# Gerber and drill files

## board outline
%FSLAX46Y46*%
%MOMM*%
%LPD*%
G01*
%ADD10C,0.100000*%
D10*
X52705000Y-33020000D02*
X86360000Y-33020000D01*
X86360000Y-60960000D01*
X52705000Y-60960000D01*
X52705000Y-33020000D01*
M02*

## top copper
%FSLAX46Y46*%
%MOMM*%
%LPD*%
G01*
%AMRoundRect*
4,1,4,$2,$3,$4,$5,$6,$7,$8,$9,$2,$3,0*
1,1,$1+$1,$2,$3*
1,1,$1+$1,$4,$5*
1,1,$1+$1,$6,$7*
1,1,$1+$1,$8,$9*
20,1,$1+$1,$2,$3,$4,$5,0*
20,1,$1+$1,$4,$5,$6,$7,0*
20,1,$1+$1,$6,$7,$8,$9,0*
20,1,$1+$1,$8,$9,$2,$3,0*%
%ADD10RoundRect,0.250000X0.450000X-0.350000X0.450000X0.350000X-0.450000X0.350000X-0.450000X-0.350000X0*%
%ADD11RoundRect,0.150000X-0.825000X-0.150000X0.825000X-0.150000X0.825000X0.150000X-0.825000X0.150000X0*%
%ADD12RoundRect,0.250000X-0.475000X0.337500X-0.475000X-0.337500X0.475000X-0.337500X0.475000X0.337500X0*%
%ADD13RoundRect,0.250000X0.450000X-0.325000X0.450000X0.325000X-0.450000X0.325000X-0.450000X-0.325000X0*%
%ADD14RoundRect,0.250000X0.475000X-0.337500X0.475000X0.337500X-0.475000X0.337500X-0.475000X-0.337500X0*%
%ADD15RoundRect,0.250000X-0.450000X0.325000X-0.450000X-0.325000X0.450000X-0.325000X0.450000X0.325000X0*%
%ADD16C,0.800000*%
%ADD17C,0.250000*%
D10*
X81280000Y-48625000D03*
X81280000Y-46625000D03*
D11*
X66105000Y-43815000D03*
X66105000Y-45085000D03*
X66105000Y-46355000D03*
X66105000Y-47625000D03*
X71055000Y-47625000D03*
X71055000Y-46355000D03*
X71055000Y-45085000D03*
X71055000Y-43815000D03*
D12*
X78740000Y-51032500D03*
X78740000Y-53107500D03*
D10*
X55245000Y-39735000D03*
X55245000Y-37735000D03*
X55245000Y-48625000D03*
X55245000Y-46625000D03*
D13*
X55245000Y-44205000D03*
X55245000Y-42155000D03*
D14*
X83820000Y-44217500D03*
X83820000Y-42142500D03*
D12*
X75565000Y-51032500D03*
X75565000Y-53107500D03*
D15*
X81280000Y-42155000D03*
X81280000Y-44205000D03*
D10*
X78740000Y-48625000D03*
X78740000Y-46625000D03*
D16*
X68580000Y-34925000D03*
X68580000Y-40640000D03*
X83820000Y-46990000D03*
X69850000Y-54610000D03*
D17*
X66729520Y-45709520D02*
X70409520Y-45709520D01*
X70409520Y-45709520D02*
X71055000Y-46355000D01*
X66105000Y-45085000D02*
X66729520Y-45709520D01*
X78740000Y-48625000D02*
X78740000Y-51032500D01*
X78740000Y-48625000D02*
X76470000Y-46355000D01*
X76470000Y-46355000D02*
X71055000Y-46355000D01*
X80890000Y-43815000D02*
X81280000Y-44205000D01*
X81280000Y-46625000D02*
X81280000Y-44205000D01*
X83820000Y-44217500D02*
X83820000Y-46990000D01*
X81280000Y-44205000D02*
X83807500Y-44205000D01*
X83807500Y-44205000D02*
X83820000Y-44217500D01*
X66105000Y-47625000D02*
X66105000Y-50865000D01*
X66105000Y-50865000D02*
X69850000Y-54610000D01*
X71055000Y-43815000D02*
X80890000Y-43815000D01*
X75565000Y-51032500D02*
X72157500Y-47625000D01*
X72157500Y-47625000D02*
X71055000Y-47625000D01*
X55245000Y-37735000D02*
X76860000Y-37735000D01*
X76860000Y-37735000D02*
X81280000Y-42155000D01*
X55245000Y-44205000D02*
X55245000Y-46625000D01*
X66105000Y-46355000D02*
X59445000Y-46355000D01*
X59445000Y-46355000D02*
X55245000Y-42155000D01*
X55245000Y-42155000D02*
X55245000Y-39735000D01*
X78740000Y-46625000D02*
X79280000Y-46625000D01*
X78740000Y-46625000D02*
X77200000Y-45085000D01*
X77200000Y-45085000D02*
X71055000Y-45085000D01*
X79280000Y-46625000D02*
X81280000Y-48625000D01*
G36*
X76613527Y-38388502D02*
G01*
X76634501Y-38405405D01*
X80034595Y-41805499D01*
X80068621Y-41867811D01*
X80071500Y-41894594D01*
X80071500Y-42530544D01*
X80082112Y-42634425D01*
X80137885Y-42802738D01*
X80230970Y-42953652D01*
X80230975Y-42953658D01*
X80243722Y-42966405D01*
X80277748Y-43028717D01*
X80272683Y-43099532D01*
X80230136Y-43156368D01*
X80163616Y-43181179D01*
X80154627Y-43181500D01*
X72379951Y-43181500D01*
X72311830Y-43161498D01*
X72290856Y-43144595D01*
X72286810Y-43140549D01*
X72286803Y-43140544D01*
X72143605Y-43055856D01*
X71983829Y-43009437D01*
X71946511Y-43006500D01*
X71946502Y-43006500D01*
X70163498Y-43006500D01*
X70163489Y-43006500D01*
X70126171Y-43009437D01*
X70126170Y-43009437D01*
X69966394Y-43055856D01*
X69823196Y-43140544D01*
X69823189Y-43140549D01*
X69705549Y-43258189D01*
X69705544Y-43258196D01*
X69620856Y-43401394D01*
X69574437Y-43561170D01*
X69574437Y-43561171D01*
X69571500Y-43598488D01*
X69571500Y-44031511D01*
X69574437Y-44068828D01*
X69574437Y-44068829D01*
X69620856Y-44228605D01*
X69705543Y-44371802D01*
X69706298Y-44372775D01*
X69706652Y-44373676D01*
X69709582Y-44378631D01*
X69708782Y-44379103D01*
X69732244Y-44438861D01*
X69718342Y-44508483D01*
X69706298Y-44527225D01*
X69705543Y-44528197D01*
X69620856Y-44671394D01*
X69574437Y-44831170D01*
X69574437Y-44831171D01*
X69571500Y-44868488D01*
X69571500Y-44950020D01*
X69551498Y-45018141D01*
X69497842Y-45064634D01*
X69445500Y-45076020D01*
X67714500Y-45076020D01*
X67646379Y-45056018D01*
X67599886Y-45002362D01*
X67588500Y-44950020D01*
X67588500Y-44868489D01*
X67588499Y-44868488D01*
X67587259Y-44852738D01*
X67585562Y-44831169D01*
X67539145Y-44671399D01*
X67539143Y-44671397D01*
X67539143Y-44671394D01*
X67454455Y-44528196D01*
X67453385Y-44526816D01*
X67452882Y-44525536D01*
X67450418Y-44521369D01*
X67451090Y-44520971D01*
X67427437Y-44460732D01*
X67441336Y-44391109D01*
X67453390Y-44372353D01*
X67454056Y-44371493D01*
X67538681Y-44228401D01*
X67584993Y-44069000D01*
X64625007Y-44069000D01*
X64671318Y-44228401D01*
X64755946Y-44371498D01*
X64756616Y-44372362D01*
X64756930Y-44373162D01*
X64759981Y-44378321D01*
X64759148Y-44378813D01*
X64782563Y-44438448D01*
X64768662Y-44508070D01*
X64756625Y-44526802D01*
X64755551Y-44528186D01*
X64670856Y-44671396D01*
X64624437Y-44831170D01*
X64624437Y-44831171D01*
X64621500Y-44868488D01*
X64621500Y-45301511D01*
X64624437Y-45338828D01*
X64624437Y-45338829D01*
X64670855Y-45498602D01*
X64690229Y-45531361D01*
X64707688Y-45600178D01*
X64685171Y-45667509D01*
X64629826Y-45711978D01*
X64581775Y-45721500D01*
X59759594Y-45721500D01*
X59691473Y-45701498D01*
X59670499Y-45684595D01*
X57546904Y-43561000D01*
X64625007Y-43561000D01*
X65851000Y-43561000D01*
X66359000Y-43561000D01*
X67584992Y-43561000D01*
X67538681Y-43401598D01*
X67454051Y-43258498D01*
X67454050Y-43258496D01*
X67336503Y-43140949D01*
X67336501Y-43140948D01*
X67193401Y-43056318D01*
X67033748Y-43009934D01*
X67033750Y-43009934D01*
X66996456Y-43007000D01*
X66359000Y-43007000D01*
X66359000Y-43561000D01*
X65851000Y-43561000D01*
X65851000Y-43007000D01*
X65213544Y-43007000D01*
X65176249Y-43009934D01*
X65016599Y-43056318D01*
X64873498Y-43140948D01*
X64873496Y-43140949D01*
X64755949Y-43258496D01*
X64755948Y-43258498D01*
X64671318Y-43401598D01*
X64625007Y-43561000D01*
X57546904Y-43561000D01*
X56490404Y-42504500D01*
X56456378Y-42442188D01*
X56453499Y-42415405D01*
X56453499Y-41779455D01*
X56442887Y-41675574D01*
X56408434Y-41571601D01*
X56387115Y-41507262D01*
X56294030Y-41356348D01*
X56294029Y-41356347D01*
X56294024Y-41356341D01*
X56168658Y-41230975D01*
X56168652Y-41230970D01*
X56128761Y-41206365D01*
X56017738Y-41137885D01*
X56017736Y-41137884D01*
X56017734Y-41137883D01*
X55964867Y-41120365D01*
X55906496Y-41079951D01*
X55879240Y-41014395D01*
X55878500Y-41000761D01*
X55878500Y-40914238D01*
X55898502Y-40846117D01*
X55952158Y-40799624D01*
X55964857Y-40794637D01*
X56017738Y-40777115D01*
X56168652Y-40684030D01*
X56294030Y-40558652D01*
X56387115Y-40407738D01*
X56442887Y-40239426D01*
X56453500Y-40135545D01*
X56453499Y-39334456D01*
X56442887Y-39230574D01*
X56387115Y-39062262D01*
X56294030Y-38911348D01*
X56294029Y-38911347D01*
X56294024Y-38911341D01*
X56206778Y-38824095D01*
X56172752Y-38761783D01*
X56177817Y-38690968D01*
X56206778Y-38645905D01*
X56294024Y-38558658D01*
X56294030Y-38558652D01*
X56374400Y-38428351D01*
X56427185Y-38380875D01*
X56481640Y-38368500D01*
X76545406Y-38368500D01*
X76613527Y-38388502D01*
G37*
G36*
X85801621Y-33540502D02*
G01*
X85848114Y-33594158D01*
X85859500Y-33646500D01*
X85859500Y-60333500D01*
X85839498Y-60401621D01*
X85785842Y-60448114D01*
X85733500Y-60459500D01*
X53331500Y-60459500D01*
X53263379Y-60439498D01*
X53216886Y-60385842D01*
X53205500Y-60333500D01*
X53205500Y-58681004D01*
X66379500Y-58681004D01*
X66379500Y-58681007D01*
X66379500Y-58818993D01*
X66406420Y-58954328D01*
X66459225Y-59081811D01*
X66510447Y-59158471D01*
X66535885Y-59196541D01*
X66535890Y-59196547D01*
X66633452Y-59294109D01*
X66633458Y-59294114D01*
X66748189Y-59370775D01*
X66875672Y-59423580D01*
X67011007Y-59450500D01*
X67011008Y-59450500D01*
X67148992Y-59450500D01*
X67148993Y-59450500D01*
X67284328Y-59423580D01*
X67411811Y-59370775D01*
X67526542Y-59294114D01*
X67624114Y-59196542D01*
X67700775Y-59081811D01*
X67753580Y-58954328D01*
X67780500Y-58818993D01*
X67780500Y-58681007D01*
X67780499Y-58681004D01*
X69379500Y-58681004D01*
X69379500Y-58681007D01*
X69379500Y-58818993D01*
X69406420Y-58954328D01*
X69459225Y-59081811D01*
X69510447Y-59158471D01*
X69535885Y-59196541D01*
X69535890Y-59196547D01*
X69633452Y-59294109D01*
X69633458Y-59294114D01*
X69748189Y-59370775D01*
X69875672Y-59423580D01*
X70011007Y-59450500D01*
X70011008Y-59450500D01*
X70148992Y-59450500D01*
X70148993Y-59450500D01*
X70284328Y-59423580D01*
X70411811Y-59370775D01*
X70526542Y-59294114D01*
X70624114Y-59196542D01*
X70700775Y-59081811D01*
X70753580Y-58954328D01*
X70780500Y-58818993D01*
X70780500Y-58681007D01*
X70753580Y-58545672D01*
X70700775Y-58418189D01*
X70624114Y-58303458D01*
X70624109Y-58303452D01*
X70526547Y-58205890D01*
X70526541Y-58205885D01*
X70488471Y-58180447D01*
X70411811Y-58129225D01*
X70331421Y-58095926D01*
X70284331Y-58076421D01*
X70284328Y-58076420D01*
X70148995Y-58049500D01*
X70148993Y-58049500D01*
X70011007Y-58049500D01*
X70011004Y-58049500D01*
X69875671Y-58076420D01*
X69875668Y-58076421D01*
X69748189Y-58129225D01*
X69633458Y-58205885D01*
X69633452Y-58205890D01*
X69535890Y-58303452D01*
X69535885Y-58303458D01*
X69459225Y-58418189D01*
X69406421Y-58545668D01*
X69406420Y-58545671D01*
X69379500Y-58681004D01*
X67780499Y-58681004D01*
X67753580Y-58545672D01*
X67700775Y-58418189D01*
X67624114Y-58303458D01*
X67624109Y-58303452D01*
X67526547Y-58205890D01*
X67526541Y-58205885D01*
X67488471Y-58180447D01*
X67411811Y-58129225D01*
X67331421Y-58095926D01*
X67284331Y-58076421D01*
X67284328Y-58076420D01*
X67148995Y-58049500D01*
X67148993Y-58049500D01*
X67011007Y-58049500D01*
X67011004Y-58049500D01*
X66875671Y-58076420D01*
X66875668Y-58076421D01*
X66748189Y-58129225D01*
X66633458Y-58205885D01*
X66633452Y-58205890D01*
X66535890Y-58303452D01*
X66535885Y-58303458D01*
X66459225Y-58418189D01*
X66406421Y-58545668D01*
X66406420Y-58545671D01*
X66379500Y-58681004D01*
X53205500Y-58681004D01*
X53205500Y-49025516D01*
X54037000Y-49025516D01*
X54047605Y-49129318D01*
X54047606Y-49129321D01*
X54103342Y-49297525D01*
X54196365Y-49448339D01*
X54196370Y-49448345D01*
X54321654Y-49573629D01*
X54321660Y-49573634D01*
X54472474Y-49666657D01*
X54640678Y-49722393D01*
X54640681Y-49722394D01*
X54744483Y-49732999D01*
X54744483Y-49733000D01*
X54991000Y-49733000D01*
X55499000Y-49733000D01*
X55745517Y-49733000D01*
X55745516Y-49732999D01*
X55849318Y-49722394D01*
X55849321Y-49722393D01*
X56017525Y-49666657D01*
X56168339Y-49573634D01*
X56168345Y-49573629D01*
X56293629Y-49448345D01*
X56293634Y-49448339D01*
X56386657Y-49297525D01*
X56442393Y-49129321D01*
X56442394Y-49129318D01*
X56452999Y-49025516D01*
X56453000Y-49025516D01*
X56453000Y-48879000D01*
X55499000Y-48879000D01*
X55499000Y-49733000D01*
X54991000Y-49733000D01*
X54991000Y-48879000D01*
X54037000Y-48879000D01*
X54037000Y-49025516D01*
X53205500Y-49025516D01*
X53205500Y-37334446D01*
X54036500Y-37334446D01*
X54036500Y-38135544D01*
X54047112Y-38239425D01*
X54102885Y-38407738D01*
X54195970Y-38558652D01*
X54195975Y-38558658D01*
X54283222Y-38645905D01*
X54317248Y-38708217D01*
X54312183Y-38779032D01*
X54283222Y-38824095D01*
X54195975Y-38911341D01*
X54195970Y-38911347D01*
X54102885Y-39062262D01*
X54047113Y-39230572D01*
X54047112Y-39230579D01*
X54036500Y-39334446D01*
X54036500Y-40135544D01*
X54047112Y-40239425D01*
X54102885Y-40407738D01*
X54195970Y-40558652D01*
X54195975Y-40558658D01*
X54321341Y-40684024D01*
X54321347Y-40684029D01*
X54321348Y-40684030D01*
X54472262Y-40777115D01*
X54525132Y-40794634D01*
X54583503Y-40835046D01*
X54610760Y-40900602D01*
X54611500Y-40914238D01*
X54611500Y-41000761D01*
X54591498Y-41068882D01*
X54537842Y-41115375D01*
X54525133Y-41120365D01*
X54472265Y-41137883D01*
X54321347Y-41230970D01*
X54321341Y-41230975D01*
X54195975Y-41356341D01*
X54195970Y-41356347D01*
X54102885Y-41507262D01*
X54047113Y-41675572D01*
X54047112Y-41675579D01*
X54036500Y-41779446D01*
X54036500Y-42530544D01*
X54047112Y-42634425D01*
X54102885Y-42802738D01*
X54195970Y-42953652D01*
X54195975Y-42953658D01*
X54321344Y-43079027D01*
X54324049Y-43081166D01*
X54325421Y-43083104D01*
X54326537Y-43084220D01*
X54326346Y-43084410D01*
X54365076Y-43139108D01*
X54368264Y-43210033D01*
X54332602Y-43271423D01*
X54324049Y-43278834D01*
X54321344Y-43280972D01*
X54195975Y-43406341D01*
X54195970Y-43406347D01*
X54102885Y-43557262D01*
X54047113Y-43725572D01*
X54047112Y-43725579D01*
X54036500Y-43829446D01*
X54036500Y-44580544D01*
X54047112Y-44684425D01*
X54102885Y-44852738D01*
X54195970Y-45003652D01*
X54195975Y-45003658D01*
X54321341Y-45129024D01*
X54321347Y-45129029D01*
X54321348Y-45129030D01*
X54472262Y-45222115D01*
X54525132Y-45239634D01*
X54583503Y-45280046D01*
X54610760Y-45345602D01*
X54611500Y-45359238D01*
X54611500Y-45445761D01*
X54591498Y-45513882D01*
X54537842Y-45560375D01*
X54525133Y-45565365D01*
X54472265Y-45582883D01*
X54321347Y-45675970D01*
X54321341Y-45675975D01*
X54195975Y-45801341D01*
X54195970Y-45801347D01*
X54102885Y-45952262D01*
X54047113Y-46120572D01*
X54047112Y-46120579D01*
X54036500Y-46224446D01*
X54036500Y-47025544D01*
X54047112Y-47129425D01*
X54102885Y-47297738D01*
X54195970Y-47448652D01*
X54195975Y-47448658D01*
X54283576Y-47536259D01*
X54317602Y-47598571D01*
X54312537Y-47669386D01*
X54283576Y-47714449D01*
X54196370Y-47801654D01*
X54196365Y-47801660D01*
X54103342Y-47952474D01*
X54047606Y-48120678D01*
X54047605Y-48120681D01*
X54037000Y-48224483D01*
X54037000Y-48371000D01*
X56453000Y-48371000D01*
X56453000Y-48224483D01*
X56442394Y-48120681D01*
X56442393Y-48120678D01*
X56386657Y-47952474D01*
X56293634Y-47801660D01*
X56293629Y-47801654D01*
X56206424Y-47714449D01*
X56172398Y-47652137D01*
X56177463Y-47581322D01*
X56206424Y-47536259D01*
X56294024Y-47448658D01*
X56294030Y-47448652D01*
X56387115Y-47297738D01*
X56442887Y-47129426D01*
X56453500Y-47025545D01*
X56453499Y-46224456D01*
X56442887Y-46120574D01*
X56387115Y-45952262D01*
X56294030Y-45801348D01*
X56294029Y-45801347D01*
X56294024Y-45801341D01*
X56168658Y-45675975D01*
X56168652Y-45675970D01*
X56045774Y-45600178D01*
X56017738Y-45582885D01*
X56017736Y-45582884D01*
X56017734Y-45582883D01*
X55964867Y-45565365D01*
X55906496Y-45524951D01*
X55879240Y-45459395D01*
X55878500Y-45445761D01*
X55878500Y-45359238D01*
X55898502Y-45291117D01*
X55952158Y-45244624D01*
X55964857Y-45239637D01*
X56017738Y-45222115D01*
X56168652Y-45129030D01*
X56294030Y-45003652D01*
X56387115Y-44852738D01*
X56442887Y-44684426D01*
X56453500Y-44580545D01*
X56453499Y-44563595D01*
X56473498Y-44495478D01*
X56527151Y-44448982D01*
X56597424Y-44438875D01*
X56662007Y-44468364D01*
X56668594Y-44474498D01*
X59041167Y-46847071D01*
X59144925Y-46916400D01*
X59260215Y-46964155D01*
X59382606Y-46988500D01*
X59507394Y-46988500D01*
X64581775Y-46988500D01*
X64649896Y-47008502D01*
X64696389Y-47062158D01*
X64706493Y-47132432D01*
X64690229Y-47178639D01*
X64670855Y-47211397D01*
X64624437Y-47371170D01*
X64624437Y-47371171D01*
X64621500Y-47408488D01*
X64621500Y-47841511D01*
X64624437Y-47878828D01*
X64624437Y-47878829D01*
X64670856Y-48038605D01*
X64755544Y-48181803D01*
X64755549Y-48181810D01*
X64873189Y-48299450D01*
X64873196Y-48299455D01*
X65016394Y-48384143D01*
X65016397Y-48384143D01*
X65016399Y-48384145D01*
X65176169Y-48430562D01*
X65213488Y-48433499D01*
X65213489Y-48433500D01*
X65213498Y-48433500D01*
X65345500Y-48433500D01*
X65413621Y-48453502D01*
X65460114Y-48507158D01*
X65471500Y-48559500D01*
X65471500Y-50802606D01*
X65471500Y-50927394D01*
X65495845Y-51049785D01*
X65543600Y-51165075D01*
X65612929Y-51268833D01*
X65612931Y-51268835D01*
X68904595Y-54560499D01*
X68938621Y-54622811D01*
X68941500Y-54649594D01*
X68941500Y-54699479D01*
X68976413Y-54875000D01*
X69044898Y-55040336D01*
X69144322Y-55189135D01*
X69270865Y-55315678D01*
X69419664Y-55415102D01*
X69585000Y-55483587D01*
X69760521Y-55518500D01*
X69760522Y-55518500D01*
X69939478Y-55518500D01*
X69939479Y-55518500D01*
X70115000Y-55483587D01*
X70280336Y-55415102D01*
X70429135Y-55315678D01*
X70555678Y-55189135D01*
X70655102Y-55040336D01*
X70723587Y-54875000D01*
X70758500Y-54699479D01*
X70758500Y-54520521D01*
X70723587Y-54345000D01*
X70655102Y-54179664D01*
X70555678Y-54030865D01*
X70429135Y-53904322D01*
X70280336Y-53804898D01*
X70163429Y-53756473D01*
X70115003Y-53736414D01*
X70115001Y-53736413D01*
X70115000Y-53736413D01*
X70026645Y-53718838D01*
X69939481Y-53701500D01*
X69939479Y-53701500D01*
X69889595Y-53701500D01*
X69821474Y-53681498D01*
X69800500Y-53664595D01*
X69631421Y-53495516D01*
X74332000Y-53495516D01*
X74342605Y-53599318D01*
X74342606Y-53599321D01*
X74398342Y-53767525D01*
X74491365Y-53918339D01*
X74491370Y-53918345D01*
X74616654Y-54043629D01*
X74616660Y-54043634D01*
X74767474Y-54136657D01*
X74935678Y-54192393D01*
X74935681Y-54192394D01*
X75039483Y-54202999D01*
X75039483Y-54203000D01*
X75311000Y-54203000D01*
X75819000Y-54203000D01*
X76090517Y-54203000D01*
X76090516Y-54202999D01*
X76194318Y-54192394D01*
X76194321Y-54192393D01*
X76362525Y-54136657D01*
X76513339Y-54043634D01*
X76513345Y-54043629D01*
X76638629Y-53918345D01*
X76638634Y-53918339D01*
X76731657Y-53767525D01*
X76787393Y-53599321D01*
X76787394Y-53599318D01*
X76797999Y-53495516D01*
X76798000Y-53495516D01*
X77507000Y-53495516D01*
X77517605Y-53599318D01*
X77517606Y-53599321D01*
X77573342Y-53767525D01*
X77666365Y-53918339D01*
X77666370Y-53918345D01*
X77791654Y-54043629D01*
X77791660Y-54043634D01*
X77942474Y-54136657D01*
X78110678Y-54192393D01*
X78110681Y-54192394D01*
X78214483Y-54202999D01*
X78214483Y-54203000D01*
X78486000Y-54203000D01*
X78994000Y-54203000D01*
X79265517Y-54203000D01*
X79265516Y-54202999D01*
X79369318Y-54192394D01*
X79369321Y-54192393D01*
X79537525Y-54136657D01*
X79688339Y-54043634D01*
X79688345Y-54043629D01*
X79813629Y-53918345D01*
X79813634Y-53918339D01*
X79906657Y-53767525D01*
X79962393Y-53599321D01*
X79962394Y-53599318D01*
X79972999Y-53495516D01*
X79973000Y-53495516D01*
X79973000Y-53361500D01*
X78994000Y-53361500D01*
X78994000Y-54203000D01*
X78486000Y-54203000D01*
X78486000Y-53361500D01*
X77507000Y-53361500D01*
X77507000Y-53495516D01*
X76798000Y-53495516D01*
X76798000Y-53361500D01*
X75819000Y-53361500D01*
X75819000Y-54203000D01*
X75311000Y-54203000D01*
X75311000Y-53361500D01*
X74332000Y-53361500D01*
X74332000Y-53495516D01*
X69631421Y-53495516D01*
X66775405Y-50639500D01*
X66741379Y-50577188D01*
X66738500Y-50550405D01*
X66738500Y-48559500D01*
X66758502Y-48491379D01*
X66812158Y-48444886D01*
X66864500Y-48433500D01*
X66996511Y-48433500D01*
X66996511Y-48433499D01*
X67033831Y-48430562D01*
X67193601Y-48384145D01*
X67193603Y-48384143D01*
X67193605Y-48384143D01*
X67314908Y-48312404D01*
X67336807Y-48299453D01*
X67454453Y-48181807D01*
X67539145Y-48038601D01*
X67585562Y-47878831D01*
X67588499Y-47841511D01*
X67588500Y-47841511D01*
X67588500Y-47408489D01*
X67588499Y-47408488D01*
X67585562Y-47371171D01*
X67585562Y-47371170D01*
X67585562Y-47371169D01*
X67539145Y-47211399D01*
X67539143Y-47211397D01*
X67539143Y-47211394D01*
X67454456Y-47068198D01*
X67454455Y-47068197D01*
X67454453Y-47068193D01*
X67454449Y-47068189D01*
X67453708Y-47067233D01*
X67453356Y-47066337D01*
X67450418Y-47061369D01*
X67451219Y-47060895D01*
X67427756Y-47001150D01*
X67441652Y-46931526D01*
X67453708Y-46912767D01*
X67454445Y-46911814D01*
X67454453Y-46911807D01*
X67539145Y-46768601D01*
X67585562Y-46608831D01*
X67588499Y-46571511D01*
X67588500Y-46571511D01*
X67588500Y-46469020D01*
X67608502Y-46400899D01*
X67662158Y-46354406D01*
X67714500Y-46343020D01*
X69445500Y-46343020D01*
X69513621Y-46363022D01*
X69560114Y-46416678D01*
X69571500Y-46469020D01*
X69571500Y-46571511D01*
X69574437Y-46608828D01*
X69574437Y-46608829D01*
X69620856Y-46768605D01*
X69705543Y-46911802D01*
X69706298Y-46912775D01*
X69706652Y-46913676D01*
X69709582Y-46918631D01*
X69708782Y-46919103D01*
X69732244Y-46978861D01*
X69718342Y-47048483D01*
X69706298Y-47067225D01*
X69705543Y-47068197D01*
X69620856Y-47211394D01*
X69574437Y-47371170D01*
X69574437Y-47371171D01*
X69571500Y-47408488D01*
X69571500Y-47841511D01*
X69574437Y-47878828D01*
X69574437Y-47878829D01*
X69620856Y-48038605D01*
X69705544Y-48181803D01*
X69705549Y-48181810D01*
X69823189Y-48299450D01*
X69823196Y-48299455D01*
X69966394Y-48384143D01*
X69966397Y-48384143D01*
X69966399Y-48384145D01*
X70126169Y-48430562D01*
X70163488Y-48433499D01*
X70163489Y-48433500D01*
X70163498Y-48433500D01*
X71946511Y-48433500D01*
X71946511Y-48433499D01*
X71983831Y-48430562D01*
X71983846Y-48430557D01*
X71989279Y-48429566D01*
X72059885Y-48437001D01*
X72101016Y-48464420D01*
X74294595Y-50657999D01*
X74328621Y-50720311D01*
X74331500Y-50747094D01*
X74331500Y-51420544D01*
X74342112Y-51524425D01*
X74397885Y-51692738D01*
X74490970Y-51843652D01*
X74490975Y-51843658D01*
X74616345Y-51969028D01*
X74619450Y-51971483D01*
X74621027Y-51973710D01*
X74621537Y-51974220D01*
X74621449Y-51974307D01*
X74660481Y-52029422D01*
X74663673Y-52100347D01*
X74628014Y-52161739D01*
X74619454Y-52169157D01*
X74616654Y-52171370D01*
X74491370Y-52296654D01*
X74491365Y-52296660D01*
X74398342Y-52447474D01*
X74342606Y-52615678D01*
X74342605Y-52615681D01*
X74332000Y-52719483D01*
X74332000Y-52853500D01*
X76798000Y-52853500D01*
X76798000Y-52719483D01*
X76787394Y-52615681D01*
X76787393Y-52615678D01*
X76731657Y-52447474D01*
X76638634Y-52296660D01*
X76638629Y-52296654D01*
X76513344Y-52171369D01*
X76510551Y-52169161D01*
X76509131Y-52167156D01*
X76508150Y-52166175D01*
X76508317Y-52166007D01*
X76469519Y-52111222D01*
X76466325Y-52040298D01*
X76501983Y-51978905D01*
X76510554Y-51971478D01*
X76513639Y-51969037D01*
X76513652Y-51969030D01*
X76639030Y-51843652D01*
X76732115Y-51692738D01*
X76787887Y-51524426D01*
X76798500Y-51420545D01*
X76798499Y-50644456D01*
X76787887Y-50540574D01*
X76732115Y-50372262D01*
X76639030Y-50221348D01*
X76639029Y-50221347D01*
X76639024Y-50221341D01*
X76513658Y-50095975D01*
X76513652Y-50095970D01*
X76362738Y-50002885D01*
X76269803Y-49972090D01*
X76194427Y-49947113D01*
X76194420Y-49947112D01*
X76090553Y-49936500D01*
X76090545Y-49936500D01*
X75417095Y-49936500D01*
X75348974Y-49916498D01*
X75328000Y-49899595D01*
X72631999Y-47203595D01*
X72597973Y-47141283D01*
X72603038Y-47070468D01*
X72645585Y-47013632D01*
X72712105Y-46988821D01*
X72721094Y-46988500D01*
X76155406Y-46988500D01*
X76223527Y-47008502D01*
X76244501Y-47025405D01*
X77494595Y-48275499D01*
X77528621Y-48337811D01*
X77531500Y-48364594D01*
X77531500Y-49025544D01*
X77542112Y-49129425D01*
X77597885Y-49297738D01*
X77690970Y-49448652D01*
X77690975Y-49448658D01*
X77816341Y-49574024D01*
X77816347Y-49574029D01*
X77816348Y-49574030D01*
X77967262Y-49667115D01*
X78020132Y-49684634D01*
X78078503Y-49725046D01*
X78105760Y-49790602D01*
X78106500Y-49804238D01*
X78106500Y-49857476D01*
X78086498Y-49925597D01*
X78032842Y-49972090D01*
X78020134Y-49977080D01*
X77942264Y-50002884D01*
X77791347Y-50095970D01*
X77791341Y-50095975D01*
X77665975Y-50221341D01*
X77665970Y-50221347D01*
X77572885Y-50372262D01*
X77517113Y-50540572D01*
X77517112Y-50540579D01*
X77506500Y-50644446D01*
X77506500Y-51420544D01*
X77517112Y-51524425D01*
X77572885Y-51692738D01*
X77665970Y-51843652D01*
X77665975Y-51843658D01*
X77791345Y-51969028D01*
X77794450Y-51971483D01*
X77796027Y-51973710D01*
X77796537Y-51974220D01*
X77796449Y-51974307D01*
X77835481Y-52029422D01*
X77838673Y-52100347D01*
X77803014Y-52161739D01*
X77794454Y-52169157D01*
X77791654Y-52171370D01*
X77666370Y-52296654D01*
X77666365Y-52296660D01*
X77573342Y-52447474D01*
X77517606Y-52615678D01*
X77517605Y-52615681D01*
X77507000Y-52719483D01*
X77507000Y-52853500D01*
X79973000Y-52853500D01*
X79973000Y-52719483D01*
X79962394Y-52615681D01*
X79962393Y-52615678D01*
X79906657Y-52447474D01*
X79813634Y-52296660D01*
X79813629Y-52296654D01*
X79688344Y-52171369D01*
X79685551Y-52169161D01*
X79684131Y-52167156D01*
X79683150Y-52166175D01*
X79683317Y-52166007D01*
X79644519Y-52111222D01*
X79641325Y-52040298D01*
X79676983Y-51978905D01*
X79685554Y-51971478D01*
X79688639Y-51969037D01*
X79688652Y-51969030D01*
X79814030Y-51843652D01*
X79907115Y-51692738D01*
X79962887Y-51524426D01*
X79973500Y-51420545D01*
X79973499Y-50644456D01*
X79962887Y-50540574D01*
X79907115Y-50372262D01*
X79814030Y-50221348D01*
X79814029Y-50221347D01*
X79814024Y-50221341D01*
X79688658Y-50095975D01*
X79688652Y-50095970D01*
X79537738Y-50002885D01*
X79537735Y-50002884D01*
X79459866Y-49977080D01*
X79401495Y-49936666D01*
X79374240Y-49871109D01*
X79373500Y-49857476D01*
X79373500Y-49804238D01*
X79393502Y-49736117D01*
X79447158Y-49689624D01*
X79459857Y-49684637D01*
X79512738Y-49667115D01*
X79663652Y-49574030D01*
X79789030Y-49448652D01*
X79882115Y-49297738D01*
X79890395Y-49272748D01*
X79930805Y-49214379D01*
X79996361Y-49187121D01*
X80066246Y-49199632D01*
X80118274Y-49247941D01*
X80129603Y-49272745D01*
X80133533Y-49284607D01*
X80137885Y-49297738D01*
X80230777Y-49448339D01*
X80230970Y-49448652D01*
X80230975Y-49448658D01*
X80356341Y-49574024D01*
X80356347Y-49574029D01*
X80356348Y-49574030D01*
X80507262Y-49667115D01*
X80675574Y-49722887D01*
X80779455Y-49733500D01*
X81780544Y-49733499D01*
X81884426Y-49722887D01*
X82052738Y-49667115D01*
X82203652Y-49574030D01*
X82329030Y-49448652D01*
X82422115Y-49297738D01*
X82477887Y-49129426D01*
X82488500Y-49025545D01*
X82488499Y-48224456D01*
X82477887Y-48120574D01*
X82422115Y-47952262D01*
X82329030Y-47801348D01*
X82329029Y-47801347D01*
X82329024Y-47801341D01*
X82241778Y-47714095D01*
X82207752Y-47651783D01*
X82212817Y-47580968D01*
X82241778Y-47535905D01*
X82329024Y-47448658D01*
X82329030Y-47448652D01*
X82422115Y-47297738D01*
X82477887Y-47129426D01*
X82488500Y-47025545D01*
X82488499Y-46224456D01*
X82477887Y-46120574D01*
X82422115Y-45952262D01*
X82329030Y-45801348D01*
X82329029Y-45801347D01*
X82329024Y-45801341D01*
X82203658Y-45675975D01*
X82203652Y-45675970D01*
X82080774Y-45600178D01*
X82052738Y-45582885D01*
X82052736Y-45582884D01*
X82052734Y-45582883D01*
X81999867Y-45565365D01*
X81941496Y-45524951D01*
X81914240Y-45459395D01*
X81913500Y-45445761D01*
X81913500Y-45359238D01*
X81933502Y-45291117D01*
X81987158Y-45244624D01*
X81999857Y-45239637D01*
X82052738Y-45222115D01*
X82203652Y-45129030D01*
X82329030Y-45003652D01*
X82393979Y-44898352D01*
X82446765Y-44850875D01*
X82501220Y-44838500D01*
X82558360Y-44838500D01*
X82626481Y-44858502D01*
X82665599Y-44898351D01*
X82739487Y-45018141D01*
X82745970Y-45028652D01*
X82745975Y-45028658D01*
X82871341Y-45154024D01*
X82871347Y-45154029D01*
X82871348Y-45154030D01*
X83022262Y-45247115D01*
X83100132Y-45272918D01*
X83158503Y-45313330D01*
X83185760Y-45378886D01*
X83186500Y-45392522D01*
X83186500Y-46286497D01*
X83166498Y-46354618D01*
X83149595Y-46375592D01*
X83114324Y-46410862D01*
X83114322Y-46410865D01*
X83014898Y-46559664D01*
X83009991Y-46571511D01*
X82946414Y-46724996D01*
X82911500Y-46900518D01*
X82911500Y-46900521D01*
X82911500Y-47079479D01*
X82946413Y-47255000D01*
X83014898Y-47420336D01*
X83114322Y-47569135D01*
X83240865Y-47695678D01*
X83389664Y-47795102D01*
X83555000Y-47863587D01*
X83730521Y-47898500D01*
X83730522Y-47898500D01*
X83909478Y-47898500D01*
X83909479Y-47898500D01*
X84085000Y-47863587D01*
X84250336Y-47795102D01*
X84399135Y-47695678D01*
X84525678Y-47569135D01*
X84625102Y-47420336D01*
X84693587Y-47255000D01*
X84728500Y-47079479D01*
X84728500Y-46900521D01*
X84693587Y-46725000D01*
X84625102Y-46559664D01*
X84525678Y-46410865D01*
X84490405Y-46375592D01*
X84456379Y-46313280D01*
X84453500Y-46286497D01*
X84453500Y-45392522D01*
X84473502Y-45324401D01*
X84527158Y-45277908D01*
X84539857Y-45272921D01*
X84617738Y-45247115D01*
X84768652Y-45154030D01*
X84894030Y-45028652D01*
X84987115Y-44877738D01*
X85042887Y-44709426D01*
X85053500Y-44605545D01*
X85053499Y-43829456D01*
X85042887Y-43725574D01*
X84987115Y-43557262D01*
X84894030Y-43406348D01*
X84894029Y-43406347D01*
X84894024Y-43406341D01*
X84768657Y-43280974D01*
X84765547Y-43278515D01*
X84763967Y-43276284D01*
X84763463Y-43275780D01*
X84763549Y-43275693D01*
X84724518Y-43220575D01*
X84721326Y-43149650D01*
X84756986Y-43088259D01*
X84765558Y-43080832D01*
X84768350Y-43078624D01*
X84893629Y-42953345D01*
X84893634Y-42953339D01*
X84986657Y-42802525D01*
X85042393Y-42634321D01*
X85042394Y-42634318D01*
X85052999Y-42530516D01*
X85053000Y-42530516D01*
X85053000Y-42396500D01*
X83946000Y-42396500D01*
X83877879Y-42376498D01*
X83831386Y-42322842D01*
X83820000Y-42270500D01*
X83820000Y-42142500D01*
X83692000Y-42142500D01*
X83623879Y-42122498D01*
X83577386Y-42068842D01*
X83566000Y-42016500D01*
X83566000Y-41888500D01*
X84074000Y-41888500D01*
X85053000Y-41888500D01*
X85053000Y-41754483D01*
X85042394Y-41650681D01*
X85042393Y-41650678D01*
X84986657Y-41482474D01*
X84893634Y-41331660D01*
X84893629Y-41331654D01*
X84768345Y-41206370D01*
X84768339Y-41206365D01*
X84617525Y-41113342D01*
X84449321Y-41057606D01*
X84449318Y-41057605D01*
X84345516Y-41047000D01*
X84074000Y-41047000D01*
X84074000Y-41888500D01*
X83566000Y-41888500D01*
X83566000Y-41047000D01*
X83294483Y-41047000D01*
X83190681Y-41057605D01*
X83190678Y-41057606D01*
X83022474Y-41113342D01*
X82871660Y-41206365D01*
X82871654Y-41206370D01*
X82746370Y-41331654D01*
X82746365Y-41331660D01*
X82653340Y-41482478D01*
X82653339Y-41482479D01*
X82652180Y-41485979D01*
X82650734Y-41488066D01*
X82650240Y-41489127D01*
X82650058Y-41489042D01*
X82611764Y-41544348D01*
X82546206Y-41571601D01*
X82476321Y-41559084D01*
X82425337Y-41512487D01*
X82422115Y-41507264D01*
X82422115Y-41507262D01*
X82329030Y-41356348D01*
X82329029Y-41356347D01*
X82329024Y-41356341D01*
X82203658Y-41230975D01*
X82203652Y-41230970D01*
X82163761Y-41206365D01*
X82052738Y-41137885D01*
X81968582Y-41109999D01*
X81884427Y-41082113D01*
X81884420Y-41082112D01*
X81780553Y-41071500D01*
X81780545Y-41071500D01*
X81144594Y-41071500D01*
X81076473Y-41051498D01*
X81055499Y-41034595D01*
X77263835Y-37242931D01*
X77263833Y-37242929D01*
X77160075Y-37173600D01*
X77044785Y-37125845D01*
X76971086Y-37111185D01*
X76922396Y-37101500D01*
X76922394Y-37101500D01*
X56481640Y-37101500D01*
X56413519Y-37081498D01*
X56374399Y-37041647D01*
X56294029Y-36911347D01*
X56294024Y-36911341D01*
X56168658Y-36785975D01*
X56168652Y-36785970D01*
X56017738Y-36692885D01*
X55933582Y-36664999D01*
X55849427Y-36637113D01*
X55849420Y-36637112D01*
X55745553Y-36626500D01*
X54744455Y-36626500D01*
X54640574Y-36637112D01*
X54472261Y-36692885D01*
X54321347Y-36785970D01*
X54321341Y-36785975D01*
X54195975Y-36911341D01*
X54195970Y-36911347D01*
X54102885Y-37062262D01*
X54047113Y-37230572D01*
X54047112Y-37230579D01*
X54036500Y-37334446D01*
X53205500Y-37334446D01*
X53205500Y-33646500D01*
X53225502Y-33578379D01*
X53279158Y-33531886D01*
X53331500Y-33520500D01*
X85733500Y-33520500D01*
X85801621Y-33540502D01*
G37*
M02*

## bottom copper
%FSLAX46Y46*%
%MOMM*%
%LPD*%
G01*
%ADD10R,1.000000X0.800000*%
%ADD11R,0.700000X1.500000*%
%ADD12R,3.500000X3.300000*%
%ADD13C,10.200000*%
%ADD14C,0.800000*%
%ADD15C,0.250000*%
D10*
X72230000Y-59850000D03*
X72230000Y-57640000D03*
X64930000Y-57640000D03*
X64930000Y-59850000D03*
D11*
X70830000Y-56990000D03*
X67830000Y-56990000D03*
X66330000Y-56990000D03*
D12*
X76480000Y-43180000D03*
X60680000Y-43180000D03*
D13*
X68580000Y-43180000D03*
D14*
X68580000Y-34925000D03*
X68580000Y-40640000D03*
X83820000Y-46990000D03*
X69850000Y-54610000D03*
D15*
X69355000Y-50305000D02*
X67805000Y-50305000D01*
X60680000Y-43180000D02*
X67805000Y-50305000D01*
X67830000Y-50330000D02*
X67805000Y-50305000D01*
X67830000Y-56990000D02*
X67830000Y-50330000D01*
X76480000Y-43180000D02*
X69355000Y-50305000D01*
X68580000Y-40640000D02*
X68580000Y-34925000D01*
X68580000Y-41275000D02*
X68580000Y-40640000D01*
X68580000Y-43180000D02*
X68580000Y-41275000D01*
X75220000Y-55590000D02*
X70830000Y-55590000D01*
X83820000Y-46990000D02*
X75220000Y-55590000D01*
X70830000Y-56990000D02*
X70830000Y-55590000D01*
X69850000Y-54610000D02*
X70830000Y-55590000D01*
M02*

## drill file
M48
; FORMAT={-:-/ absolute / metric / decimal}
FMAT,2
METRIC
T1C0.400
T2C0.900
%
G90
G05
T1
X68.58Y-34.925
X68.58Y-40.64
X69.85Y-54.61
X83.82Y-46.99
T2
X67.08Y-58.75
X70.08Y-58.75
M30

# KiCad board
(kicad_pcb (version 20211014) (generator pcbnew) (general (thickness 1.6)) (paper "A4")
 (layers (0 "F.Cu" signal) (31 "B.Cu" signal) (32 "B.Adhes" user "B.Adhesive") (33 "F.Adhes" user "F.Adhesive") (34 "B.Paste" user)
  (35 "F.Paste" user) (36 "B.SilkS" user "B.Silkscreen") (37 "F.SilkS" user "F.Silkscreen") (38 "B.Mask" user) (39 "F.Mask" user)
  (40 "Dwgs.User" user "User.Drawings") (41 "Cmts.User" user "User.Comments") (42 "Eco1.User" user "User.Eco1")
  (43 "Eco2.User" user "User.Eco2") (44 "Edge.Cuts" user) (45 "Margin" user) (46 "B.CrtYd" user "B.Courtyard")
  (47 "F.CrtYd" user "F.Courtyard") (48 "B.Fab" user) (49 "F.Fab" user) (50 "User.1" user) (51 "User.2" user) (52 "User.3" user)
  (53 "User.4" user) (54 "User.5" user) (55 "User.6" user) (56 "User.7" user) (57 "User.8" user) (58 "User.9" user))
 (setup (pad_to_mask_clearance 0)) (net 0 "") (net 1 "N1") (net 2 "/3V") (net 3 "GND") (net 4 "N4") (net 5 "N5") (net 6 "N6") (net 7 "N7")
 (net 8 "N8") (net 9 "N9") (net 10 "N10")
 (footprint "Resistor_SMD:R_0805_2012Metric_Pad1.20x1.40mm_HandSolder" (layer "F.Cu") (at 81.28 47.625 90)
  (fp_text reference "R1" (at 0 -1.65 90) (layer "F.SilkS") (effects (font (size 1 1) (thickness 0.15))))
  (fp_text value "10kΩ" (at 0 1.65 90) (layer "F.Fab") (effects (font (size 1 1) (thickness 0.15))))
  (pad "1" smd roundrect (at -1 0 90) (size 1.2 1.4) (layers "F.Cu" "F.Paste" "F.Mask") (roundrect_rratio 0.208333) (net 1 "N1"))
  (pad "2" smd roundrect (at 1 0 90) (size 1.2 1.4) (layers "F.Cu" "F.Paste" "F.Mask") (roundrect_rratio 0.208333) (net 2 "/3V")))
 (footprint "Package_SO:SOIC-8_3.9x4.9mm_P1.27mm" (layer "F.Cu") (at 68.58 45.72)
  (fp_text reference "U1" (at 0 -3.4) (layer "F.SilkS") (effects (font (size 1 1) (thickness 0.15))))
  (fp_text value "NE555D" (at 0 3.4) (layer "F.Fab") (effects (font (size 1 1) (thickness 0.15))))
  (pad "1" smd roundrect (at -2.475 -1.905) (size 1.95 0.6) (layers "F.Cu" "F.Paste" "F.Mask") (roundrect_rratio 0.25) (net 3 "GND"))
  (pad "2" smd roundrect (at -2.475 -0.635) (size 1.95 0.6) (layers "F.Cu" "F.Paste" "F.Mask") (roundrect_rratio 0.25) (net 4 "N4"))
  (pad "3" smd roundrect (at -2.475 0.635) (size 1.95 0.6) (layers "F.Cu" "F.Paste" "F.Mask") (roundrect_rratio 0.25) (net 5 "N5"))
  (pad "4" smd roundrect (at -2.475 1.905) (size 1.95 0.6) (layers "F.Cu" "F.Paste" "F.Mask") (roundrect_rratio 0.25) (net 2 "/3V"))
  (pad "5" smd roundrect (at 2.475 1.905) (size 1.95 0.6) (layers "F.Cu" "F.Paste" "F.Mask") (roundrect_rratio 0.25) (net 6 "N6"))
  (pad "6" smd roundrect (at 2.475 0.635) (size 1.95 0.6) (layers "F.Cu" "F.Paste" "F.Mask") (roundrect_rratio 0.25) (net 4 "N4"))
  (pad "7" smd roundrect (at 2.475 -0.635) (size 1.95 0.6) (layers "F.Cu" "F.Paste" "F.Mask") (roundrect_rratio 0.25) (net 1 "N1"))
  (pad "8" smd roundrect (at 2.475 -1.905) (size 1.95 0.6) (layers "F.Cu" "F.Paste" "F.Mask") (roundrect_rratio 0.25) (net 2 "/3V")))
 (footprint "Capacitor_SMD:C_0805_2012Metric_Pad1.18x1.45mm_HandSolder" (layer "F.Cu") (at 78.74 52.07 -90)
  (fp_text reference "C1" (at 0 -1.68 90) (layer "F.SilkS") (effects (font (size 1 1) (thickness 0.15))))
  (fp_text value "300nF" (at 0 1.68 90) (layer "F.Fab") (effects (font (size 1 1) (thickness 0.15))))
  (pad "1" smd roundrect (at -1.0375 0 270) (size 1.175 1.45) (layers "F.Cu" "F.Paste" "F.Mask") (roundrect_rratio 0.212766) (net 4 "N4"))
  (pad "2" smd roundrect (at 1.0375 0 270) (size 1.175 1.45) (layers "F.Cu" "F.Paste" "F.Mask") (roundrect_rratio 0.212766) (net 3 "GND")))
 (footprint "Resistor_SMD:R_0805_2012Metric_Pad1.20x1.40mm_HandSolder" (layer "F.Cu") (at 55.245 38.735 90)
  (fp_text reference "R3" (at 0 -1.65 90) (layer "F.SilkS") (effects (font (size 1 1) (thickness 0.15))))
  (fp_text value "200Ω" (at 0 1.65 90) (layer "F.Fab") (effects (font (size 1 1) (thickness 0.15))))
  (pad "1" smd roundrect (at -1 0 90) (size 1.2 1.4) (layers "F.Cu" "F.Paste" "F.Mask") (roundrect_rratio 0.208333) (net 5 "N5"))
  (pad "2" smd roundrect (at 1 0 90) (size 1.2 1.4) (layers "F.Cu" "F.Paste" "F.Mask") (roundrect_rratio 0.208333) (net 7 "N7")))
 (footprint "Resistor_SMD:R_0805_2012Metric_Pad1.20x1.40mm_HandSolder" (layer "F.Cu") (at 55.245 47.625 90)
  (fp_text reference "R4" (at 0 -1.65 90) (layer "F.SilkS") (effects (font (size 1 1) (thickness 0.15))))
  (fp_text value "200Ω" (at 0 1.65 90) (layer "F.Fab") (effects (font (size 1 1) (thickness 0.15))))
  (pad "1" smd roundrect (at -1 0 90) (size 1.2 1.4) (layers "F.Cu" "F.Paste" "F.Mask") (roundrect_rratio 0.208333) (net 3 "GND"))
  (pad "2" smd roundrect (at 1 0 90) (size 1.2 1.4) (layers "F.Cu" "F.Paste" "F.Mask") (roundrect_rratio 0.208333) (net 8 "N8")))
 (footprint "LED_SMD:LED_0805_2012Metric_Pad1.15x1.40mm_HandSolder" (layer "F.Cu") (at 55.245 43.18 90)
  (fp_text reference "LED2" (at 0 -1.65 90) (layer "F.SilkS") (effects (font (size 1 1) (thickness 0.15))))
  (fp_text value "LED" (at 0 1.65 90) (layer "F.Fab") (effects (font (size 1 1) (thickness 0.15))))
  (pad "1" smd roundrect (at -1.025 0 90) (size 1.15 1.4) (layers "F.Cu" "F.Paste" "F.Mask") (roundrect_rratio 0.217391) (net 8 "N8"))
  (pad "2" smd roundrect (at 1.025 0 90) (size 1.15 1.4) (layers "F.Cu" "F.Paste" "F.Mask") (roundrect_rratio 0.217391) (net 5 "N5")))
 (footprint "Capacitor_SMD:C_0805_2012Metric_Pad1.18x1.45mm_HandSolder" (layer "F.Cu") (at 83.82 43.18 90)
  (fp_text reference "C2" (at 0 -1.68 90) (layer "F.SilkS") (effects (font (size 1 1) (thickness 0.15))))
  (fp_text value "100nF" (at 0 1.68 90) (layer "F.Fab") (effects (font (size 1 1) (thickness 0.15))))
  (pad "1" smd roundrect (at -1.0375 0 90) (size 1.175 1.45) (layers "F.Cu" "F.Paste" "F.Mask") (roundrect_rratio 0.212766) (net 2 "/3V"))
  (pad "2" smd roundrect (at 1.0375 0 90) (size 1.175 1.45) (layers "F.Cu" "F.Paste" "F.Mask") (roundrect_rratio 0.212766) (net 3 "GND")))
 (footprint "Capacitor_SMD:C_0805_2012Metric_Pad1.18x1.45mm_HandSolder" (layer "F.Cu") (at 75.565 52.07 -90)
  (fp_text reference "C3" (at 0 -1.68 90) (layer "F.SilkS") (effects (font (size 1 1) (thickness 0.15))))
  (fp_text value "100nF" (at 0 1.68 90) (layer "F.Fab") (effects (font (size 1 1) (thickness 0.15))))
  (pad "1" smd roundrect (at -1.0375 0 270) (size 1.175 1.45) (layers "F.Cu" "F.Paste" "F.Mask") (roundrect_rratio 0.212766) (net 6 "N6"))
  (pad "2" smd roundrect (at 1.0375 0 270) (size 1.175 1.45) (layers "F.Cu" "F.Paste" "F.Mask") (roundrect_rratio 0.212766) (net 3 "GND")))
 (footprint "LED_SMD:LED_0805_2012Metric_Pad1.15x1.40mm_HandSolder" (layer "F.Cu") (at 81.28 43.18 -90)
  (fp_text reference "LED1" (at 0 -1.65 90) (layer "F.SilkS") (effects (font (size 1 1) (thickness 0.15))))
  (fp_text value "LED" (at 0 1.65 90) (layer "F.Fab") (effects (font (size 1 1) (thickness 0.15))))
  (pad "1" smd roundrect (at -1.025 0 270) (size 1.15 1.4) (layers "F.Cu" "F.Paste" "F.Mask") (roundrect_rratio 0.217391) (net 7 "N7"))
  (pad "2" smd roundrect (at 1.025 0 270) (size 1.15 1.4) (layers "F.Cu" "F.Paste" "F.Mask") (roundrect_rratio 0.217391) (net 2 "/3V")))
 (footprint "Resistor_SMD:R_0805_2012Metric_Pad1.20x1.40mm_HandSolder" (layer "F.Cu") (at 78.74 47.625 90)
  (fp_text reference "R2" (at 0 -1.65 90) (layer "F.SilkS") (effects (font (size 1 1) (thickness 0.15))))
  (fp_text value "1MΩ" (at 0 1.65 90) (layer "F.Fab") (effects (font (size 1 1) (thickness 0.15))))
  (pad "1" smd roundrect (at -1 0 90) (size 1.2 1.4) (layers "F.Cu" "F.Paste" "F.Mask") (roundrect_rratio 0.208333) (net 4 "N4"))
  (pad "2" smd roundrect (at 1 0 90) (size 1.2 1.4) (layers "F.Cu" "F.Paste" "F.Mask") (roundrect_rratio 0.208333) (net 1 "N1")))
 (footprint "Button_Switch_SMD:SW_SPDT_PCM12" (layer "B.Cu") (at 68.58 58.42 180)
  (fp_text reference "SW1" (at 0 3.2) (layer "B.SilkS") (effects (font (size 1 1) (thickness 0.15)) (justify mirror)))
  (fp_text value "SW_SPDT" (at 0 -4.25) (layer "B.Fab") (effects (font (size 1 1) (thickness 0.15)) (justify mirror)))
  (pad "" smd rect (at -3.65 -1.43 180) (size 1 0.8) (layers "B.Cu" "B.Paste" "B.Mask"))
  (pad "" smd rect (at -3.65 0.78 180) (size 1 0.8) (layers "B.Cu" "B.Paste" "B.Mask"))
  (pad "" np_thru_hole circle (at -1.5 -0.33 180) (size 0.9 0.9) (drill 0.9) (layers *.Cu *.Mask))
  (pad "" smd rect (at 3.65 0.78 180) (size 1 0.8) (layers "B.Cu" "B.Paste" "B.Mask"))
  (pad "" smd rect (at 3.65 -1.43 180) (size 1 0.8) (layers "B.Cu" "B.Paste" "B.Mask"))
  (pad "" np_thru_hole circle (at 1.5 -0.33 180) (size 0.9 0.9) (drill 0.9) (layers *.Cu *.Mask))
  (pad "1" smd rect (at -2.25 1.43 180) (size 0.7 1.5) (layers "B.Cu" "B.Paste" "B.Mask") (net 2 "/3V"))
  (pad "2" smd rect (at 0.75 1.43 180) (size 0.7 1.5) (layers "B.Cu" "B.Paste" "B.Mask") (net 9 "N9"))
  (pad "3" smd rect (at 2.25 1.43 180) (size 0.7 1.5) (layers "B.Cu" "B.Paste" "B.Mask") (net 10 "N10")))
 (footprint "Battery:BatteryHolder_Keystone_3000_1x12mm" (layer "B.Cu") (at 68.58 43.18 180)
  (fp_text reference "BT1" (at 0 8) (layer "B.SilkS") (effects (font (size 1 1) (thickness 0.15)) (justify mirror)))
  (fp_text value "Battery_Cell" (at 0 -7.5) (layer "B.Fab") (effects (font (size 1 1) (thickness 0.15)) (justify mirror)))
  (pad "1" smd rect (at -7.9 0 180) (size 3.5 3.3) (layers "B.Cu" "B.Paste" "B.Mask") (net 9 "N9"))
  (pad "1" smd rect (at 7.9 0 180) (size 3.5 3.3) (layers "B.Cu" "B.Paste" "B.Mask") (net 9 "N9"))
  (pad "2" smd circle (at 0 0 180) (size 10.2 10.2) (layers "B.Cu" "B.Mask") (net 3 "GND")))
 (gr_rect (start 52.705 33.02) (end 86.36 60.96) (layer "Edge.Cuts") (width 0.1) (fill none))
 (segment (start 69.355 50.305) (end 67.805 50.305) (width 0.25) (layer "B.Cu") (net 9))
 (segment (start 60.68 43.18) (end 67.805 50.305) (width 0.25) (layer "B.Cu") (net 9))
 (segment (start 67.83 50.33) (end 67.805 50.305) (width 0.25) (layer "B.Cu") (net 9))
 (segment (start 67.83 56.99) (end 67.83 50.33) (width 0.25) (layer "B.Cu") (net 9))
 (segment (start 76.48 43.18) (end 69.355 50.305) (width 0.25) (layer "B.Cu") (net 9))
 (via (at 68.58 34.925) (size 0.8) (drill 0.4) (layers "F.Cu" "B.Cu") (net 3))
 (via (at 68.58 40.64) (size 0.8) (drill 0.4) (layers "F.Cu" "B.Cu") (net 3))
 (segment (start 68.58 40.64) (end 68.58 34.925) (width 0.25) (layer "B.Cu") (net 3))
 (segment (start 68.58 41.275) (end 68.58 40.64) (width 0.25) (layer "B.Cu") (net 3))
 (segment (start 68.58 43.18) (end 68.58 41.275) (width 0.25) (layer "B.Cu") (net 3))
 (segment (start 66.72952 45.70952) (end 70.40952 45.70952) (width 0.25) (layer "F.Cu") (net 4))
 (segment (start 70.40952 45.70952) (end 71.055 46.355) (width 0.25) (layer "F.Cu") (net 4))
 (segment (start 66.105 45.085) (end 66.72952 45.70952) (width 0.25) (layer "F.Cu") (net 4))
 (segment (start 78.74 48.625) (end 78.74 51.0325) (width 0.25) (layer "F.Cu") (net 4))
 (segment (start 78.74 48.625) (end 76.47 46.355) (width 0.25) (layer "F.Cu") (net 4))
 (segment (start 76.47 46.355) (end 71.055 46.355) (width 0.25) (layer "F.Cu") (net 4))
 (segment (start 80.89 43.815) (end 81.28 44.205) (width 0.25) (layer "F.Cu") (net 2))
 (segment (start 81.28 46.625) (end 81.28 44.205) (width 0.25) (layer "F.Cu") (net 2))
 (segment (start 83.82 44.2175) (end 83.82 46.99) (width 0.25) (layer "F.Cu") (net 2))
 (segment (start 81.28 44.205) (end 83.8075 44.205) (width 0.25) (layer "F.Cu") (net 2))
 (segment (start 83.8075 44.205) (end 83.82 44.2175) (width 0.25) (layer "F.Cu") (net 2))
 (segment (start 66.105 47.625) (end 66.105 50.865) (width 0.25) (layer "F.Cu") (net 2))
 (segment (start 66.105 50.865) (end 69.85 54.61) (width 0.25) (layer "F.Cu") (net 2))
 (segment (start 71.055 43.815) (end 80.89 43.815) (width 0.25) (layer "F.Cu") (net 2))
 (via (at 83.82 46.99) (size 0.8) (drill 0.4) (layers "F.Cu" "B.Cu") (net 2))
 (via (at 69.85 54.61) (size 0.8) (drill 0.4) (layers "F.Cu" "B.Cu") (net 2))
 (segment (start 75.22 55.59) (end 70.83 55.59) (width 0.25) (layer "B.Cu") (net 2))
 (segment (start 83.82 46.99) (end 75.22 55.59) (width 0.25) (layer "B.Cu") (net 2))
 (segment (start 70.83 56.99) (end 70.83 55.59) (width 0.25) (layer "B.Cu") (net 2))
 (segment (start 69.85 54.61) (end 70.83 55.59) (width 0.25) (layer "B.Cu") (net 2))
 (segment (start 75.565 51.0325) (end 72.1575 47.625) (width 0.25) (layer "F.Cu") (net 6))
 (segment (start 72.1575 47.625) (end 71.055 47.625) (width 0.25) (layer "F.Cu") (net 6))
 (segment (start 55.245 37.735) (end 76.86 37.735) (width 0.25) (layer "F.Cu") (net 7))
 (segment (start 76.86 37.735) (end 81.28 42.155) (width 0.25) (layer "F.Cu") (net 7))
 (segment (start 55.245 44.205) (end 55.245 46.625) (width 0.25) (layer "F.Cu") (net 8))
 (segment (start 66.105 46.355) (end 59.445 46.355) (width 0.25) (layer "F.Cu") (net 5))
 (segment (start 59.445 46.355) (end 55.245 42.155) (width 0.25) (layer "F.Cu") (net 5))
 (segment (start 55.245 42.155) (end 55.245 39.735) (width 0.25) (layer "F.Cu") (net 5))
 (segment (start 78.74 46.625) (end 79.28 46.625) (width 0.25) (layer "F.Cu") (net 1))
 (segment (start 78.74 46.625) (end 77.2 45.085) (width 0.25) (layer "F.Cu") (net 1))
 (segment (start 77.2 45.085) (end 71.055 45.085) (width 0.25) (layer "F.Cu") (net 1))
 (segment (start 79.28 46.625) (end 81.28 48.625) (width 0.25) (layer "F.Cu") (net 1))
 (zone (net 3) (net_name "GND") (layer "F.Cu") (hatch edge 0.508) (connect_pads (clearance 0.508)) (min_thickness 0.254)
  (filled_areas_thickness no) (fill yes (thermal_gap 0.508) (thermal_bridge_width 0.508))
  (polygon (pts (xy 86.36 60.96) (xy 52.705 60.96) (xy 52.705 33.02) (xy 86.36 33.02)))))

